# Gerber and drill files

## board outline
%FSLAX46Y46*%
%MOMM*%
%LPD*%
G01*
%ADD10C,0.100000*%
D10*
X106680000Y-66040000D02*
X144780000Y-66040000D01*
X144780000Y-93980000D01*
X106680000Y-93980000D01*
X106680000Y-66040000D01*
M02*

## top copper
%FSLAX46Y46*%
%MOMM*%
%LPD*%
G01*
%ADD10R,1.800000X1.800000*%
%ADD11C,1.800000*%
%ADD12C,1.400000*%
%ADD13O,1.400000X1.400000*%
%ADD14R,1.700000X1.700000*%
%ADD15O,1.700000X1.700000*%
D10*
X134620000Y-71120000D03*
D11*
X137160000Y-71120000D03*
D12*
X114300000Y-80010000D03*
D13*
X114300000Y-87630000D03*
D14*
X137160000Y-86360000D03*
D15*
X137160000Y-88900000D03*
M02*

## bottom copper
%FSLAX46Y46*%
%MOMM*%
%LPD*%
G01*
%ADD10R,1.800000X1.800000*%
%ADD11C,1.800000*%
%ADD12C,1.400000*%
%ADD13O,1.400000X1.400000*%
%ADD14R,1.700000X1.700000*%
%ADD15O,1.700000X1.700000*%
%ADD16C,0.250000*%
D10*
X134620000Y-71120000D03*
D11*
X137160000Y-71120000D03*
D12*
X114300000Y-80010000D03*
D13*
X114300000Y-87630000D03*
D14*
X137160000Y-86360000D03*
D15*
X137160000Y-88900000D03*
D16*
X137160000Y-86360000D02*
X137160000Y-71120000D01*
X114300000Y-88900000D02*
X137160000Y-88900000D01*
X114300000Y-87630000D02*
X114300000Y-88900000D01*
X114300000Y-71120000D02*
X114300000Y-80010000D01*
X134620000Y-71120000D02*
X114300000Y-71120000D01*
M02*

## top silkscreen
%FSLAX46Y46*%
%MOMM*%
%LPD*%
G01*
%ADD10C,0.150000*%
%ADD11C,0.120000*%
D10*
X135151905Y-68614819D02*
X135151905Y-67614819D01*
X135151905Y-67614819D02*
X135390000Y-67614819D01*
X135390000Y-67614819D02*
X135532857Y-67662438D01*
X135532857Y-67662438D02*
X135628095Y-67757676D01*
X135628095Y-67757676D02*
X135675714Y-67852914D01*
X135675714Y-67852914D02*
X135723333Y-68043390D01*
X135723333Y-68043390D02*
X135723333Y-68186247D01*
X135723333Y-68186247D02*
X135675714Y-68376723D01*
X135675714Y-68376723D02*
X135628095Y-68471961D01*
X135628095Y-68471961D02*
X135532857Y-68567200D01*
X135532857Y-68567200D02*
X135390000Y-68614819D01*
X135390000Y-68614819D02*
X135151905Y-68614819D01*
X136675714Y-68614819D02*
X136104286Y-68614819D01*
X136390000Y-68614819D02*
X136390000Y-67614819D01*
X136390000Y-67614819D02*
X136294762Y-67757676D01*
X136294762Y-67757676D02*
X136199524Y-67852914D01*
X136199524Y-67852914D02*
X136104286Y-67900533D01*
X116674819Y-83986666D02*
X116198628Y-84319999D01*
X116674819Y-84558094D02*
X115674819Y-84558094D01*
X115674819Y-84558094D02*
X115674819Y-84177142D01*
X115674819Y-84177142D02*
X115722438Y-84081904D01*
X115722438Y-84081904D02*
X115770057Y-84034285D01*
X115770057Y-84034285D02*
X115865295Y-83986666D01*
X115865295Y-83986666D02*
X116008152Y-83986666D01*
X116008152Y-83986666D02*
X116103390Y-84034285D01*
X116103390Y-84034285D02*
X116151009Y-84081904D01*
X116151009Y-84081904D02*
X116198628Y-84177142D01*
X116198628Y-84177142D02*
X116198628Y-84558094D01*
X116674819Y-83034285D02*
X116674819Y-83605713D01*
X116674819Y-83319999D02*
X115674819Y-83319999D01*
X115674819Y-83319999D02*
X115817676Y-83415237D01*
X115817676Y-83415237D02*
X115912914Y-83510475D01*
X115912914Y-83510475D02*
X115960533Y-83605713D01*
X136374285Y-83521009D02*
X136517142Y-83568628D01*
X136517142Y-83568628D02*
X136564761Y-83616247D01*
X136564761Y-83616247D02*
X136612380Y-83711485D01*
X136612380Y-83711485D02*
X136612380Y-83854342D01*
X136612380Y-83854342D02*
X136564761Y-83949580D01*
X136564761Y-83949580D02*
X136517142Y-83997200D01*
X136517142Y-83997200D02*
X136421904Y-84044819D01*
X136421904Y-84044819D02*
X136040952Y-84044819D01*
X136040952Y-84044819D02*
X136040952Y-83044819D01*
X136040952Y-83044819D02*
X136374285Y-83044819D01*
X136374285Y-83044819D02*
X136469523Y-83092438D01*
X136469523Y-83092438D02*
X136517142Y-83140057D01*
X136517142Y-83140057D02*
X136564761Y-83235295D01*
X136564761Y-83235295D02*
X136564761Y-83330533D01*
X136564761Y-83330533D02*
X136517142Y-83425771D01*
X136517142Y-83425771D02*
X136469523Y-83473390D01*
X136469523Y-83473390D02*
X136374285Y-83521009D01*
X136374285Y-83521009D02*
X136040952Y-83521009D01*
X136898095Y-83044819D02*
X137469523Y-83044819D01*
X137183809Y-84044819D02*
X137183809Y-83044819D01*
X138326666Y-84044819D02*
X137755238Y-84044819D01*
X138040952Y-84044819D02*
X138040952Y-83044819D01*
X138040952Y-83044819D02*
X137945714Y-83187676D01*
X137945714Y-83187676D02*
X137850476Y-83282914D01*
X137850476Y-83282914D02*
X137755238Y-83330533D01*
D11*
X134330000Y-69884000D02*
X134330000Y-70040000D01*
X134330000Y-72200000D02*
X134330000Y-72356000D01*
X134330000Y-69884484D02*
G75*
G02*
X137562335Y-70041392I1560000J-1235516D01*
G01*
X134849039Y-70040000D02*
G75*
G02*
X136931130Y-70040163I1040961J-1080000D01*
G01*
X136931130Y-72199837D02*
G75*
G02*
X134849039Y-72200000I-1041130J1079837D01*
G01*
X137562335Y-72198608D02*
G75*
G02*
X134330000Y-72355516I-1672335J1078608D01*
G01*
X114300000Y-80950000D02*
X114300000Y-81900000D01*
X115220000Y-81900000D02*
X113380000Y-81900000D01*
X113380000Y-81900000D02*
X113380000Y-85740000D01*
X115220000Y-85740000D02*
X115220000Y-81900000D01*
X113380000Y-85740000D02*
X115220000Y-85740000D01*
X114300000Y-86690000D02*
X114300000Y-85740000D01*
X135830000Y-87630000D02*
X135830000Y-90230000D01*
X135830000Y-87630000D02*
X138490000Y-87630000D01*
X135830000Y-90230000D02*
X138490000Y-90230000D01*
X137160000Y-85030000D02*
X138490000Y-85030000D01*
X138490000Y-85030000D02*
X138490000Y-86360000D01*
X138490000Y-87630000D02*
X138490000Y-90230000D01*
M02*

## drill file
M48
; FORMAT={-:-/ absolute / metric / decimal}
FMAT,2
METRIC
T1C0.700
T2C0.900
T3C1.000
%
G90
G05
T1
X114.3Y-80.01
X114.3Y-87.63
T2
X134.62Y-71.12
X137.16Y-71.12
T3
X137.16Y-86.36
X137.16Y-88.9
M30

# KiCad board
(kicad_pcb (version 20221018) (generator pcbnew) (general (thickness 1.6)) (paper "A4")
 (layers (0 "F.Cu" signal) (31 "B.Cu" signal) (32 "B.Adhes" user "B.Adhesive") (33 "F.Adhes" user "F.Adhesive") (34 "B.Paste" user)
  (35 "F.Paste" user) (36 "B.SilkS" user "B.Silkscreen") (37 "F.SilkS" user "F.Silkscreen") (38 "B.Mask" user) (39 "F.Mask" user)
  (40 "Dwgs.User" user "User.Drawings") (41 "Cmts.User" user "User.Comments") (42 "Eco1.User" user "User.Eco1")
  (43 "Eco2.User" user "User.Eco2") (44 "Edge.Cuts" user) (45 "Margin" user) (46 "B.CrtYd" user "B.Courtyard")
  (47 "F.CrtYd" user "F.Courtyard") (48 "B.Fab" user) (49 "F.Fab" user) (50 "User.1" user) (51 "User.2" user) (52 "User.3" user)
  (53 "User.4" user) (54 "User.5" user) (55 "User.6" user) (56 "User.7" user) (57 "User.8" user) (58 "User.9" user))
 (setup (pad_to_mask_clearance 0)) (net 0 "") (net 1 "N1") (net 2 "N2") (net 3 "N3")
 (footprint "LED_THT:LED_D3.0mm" (layer "F.Cu") (at 134.62 71.12)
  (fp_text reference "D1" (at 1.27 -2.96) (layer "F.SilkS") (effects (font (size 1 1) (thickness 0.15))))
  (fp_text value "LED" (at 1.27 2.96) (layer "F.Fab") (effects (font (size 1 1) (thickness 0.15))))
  (fp_line (start -0.29 -1.236) (end -0.29 -1.08) (stroke (width 0.12) (type solid)) (layer "F.SilkS"))
  (fp_line (start -0.29 1.08) (end -0.29 1.236) (stroke (width 0.12) (type solid)) (layer "F.SilkS"))
  (fp_arc (start -0.29 -1.235516) (mid 1.366487 -1.987659) (end 2.942335 -1.078608) (stroke (width 0.12) (type solid)) (layer "F.SilkS"))
  (fp_arc (start 0.229039 -1.08) (mid 1.270117 -1.5) (end 2.31113 -1.079837) (stroke (width 0.12) (type solid)) (layer "F.SilkS"))
  (fp_arc (start 2.31113 1.079837) (mid 1.270117 1.5) (end 0.229039 1.08) (stroke (width 0.12) (type solid)) (layer "F.SilkS"))
  (fp_arc (start 2.942335 1.078608) (mid 1.366487 1.987659) (end -0.29 1.235516) (stroke (width 0.12) (type solid)) (layer "F.SilkS"))
  (pad "1" thru_hole rect (at 0 0) (size 1.8 1.8) (drill 0.9) (layers "*.Cu" "*.Mask") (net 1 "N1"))
  (pad "2" thru_hole circle (at 2.54 0) (size 1.8 1.8) (drill 0.9) (layers "*.Cu" "*.Mask") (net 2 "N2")))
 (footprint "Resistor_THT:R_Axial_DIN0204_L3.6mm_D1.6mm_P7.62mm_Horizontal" (layer "F.Cu") (at 114.3 80.01 -90)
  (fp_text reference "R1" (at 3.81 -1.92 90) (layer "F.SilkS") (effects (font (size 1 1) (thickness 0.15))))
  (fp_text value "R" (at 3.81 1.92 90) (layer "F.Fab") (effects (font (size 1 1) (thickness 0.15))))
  (fp_line (start 0.94 0) (end 1.89 0) (stroke (width 0.12) (type solid)) (layer "F.SilkS"))
  (fp_line (start 1.89 -0.92) (end 1.89 0.92) (stroke (width 0.12) (type solid)) (layer "F.SilkS"))
  (fp_line (start 1.89 0.92) (end 5.73 0.92) (stroke (width 0.12) (type solid)) (layer "F.SilkS"))
  (fp_line (start 5.73 -0.92) (end 1.89 -0.92) (stroke (width 0.12) (type solid)) (layer "F.SilkS"))
  (fp_line (start 5.73 0.92) (end 5.73 -0.92) (stroke (width 0.12) (type solid)) (layer "F.SilkS"))
  (fp_line (start 6.68 0) (end 5.73 0) (stroke (width 0.12) (type solid)) (layer "F.SilkS"))
  (pad "1" thru_hole circle (at 0 0 270) (size 1.4 1.4) (drill 0.7) (layers "*.Cu" "*.Mask") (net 1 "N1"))
  (pad "2" thru_hole oval (at 7.62 0 270) (size 1.4 1.4) (drill 0.7) (layers "*.Cu" "*.Mask") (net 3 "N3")))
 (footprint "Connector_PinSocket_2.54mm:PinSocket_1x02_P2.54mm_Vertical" (layer "F.Cu") (at 137.16 86.36)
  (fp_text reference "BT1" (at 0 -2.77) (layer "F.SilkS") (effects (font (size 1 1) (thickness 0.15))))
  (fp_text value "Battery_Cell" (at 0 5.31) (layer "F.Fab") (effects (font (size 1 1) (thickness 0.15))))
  (fp_line (start -1.33 1.27) (end -1.33 3.87) (stroke (width 0.12) (type solid)) (layer "F.SilkS"))
  (fp_line (start -1.33 1.27) (end 1.33 1.27) (stroke (width 0.12) (type solid)) (layer "F.SilkS"))
  (fp_line (start -1.33 3.87) (end 1.33 3.87) (stroke (width 0.12) (type solid)) (layer "F.SilkS"))
  (fp_line (start 0 -1.33) (end 1.33 -1.33) (stroke (width 0.12) (type solid)) (layer "F.SilkS"))
  (fp_line (start 1.33 -1.33) (end 1.33 0) (stroke (width 0.12) (type solid)) (layer "F.SilkS"))
  (fp_line (start 1.33 1.27) (end 1.33 3.87) (stroke (width 0.12) (type solid)) (layer "F.SilkS"))
  (pad "1" thru_hole rect (at 0 0) (size 1.7 1.7) (drill 1) (layers "*.Cu" "*.Mask") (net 2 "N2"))
  (pad "2" thru_hole oval (at 0 2.54) (size 1.7 1.7) (drill 1) (layers "*.Cu" "*.Mask") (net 3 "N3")))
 (gr_rect (start 106.68 66.04) (end 144.78 93.98) (stroke (width 0.1) (type default)) (fill none) (layer "Edge.Cuts"))
 (segment (start 137.16 86.36) (end 137.16 71.12) (width 0.25) (layer "B.Cu") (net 2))
 (segment (start 114.3 88.9) (end 137.16 88.9) (width 0.25) (layer "B.Cu") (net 3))
 (segment (start 114.3 87.63) (end 114.3 88.9) (width 0.25) (layer "B.Cu") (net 3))
 (segment (start 114.3 71.12) (end 114.3 80.01) (width 0.25) (layer "B.Cu") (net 1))
 (segment (start 134.62 71.12) (end 114.3 71.12) (width 0.25) (layer "B.Cu") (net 1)))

